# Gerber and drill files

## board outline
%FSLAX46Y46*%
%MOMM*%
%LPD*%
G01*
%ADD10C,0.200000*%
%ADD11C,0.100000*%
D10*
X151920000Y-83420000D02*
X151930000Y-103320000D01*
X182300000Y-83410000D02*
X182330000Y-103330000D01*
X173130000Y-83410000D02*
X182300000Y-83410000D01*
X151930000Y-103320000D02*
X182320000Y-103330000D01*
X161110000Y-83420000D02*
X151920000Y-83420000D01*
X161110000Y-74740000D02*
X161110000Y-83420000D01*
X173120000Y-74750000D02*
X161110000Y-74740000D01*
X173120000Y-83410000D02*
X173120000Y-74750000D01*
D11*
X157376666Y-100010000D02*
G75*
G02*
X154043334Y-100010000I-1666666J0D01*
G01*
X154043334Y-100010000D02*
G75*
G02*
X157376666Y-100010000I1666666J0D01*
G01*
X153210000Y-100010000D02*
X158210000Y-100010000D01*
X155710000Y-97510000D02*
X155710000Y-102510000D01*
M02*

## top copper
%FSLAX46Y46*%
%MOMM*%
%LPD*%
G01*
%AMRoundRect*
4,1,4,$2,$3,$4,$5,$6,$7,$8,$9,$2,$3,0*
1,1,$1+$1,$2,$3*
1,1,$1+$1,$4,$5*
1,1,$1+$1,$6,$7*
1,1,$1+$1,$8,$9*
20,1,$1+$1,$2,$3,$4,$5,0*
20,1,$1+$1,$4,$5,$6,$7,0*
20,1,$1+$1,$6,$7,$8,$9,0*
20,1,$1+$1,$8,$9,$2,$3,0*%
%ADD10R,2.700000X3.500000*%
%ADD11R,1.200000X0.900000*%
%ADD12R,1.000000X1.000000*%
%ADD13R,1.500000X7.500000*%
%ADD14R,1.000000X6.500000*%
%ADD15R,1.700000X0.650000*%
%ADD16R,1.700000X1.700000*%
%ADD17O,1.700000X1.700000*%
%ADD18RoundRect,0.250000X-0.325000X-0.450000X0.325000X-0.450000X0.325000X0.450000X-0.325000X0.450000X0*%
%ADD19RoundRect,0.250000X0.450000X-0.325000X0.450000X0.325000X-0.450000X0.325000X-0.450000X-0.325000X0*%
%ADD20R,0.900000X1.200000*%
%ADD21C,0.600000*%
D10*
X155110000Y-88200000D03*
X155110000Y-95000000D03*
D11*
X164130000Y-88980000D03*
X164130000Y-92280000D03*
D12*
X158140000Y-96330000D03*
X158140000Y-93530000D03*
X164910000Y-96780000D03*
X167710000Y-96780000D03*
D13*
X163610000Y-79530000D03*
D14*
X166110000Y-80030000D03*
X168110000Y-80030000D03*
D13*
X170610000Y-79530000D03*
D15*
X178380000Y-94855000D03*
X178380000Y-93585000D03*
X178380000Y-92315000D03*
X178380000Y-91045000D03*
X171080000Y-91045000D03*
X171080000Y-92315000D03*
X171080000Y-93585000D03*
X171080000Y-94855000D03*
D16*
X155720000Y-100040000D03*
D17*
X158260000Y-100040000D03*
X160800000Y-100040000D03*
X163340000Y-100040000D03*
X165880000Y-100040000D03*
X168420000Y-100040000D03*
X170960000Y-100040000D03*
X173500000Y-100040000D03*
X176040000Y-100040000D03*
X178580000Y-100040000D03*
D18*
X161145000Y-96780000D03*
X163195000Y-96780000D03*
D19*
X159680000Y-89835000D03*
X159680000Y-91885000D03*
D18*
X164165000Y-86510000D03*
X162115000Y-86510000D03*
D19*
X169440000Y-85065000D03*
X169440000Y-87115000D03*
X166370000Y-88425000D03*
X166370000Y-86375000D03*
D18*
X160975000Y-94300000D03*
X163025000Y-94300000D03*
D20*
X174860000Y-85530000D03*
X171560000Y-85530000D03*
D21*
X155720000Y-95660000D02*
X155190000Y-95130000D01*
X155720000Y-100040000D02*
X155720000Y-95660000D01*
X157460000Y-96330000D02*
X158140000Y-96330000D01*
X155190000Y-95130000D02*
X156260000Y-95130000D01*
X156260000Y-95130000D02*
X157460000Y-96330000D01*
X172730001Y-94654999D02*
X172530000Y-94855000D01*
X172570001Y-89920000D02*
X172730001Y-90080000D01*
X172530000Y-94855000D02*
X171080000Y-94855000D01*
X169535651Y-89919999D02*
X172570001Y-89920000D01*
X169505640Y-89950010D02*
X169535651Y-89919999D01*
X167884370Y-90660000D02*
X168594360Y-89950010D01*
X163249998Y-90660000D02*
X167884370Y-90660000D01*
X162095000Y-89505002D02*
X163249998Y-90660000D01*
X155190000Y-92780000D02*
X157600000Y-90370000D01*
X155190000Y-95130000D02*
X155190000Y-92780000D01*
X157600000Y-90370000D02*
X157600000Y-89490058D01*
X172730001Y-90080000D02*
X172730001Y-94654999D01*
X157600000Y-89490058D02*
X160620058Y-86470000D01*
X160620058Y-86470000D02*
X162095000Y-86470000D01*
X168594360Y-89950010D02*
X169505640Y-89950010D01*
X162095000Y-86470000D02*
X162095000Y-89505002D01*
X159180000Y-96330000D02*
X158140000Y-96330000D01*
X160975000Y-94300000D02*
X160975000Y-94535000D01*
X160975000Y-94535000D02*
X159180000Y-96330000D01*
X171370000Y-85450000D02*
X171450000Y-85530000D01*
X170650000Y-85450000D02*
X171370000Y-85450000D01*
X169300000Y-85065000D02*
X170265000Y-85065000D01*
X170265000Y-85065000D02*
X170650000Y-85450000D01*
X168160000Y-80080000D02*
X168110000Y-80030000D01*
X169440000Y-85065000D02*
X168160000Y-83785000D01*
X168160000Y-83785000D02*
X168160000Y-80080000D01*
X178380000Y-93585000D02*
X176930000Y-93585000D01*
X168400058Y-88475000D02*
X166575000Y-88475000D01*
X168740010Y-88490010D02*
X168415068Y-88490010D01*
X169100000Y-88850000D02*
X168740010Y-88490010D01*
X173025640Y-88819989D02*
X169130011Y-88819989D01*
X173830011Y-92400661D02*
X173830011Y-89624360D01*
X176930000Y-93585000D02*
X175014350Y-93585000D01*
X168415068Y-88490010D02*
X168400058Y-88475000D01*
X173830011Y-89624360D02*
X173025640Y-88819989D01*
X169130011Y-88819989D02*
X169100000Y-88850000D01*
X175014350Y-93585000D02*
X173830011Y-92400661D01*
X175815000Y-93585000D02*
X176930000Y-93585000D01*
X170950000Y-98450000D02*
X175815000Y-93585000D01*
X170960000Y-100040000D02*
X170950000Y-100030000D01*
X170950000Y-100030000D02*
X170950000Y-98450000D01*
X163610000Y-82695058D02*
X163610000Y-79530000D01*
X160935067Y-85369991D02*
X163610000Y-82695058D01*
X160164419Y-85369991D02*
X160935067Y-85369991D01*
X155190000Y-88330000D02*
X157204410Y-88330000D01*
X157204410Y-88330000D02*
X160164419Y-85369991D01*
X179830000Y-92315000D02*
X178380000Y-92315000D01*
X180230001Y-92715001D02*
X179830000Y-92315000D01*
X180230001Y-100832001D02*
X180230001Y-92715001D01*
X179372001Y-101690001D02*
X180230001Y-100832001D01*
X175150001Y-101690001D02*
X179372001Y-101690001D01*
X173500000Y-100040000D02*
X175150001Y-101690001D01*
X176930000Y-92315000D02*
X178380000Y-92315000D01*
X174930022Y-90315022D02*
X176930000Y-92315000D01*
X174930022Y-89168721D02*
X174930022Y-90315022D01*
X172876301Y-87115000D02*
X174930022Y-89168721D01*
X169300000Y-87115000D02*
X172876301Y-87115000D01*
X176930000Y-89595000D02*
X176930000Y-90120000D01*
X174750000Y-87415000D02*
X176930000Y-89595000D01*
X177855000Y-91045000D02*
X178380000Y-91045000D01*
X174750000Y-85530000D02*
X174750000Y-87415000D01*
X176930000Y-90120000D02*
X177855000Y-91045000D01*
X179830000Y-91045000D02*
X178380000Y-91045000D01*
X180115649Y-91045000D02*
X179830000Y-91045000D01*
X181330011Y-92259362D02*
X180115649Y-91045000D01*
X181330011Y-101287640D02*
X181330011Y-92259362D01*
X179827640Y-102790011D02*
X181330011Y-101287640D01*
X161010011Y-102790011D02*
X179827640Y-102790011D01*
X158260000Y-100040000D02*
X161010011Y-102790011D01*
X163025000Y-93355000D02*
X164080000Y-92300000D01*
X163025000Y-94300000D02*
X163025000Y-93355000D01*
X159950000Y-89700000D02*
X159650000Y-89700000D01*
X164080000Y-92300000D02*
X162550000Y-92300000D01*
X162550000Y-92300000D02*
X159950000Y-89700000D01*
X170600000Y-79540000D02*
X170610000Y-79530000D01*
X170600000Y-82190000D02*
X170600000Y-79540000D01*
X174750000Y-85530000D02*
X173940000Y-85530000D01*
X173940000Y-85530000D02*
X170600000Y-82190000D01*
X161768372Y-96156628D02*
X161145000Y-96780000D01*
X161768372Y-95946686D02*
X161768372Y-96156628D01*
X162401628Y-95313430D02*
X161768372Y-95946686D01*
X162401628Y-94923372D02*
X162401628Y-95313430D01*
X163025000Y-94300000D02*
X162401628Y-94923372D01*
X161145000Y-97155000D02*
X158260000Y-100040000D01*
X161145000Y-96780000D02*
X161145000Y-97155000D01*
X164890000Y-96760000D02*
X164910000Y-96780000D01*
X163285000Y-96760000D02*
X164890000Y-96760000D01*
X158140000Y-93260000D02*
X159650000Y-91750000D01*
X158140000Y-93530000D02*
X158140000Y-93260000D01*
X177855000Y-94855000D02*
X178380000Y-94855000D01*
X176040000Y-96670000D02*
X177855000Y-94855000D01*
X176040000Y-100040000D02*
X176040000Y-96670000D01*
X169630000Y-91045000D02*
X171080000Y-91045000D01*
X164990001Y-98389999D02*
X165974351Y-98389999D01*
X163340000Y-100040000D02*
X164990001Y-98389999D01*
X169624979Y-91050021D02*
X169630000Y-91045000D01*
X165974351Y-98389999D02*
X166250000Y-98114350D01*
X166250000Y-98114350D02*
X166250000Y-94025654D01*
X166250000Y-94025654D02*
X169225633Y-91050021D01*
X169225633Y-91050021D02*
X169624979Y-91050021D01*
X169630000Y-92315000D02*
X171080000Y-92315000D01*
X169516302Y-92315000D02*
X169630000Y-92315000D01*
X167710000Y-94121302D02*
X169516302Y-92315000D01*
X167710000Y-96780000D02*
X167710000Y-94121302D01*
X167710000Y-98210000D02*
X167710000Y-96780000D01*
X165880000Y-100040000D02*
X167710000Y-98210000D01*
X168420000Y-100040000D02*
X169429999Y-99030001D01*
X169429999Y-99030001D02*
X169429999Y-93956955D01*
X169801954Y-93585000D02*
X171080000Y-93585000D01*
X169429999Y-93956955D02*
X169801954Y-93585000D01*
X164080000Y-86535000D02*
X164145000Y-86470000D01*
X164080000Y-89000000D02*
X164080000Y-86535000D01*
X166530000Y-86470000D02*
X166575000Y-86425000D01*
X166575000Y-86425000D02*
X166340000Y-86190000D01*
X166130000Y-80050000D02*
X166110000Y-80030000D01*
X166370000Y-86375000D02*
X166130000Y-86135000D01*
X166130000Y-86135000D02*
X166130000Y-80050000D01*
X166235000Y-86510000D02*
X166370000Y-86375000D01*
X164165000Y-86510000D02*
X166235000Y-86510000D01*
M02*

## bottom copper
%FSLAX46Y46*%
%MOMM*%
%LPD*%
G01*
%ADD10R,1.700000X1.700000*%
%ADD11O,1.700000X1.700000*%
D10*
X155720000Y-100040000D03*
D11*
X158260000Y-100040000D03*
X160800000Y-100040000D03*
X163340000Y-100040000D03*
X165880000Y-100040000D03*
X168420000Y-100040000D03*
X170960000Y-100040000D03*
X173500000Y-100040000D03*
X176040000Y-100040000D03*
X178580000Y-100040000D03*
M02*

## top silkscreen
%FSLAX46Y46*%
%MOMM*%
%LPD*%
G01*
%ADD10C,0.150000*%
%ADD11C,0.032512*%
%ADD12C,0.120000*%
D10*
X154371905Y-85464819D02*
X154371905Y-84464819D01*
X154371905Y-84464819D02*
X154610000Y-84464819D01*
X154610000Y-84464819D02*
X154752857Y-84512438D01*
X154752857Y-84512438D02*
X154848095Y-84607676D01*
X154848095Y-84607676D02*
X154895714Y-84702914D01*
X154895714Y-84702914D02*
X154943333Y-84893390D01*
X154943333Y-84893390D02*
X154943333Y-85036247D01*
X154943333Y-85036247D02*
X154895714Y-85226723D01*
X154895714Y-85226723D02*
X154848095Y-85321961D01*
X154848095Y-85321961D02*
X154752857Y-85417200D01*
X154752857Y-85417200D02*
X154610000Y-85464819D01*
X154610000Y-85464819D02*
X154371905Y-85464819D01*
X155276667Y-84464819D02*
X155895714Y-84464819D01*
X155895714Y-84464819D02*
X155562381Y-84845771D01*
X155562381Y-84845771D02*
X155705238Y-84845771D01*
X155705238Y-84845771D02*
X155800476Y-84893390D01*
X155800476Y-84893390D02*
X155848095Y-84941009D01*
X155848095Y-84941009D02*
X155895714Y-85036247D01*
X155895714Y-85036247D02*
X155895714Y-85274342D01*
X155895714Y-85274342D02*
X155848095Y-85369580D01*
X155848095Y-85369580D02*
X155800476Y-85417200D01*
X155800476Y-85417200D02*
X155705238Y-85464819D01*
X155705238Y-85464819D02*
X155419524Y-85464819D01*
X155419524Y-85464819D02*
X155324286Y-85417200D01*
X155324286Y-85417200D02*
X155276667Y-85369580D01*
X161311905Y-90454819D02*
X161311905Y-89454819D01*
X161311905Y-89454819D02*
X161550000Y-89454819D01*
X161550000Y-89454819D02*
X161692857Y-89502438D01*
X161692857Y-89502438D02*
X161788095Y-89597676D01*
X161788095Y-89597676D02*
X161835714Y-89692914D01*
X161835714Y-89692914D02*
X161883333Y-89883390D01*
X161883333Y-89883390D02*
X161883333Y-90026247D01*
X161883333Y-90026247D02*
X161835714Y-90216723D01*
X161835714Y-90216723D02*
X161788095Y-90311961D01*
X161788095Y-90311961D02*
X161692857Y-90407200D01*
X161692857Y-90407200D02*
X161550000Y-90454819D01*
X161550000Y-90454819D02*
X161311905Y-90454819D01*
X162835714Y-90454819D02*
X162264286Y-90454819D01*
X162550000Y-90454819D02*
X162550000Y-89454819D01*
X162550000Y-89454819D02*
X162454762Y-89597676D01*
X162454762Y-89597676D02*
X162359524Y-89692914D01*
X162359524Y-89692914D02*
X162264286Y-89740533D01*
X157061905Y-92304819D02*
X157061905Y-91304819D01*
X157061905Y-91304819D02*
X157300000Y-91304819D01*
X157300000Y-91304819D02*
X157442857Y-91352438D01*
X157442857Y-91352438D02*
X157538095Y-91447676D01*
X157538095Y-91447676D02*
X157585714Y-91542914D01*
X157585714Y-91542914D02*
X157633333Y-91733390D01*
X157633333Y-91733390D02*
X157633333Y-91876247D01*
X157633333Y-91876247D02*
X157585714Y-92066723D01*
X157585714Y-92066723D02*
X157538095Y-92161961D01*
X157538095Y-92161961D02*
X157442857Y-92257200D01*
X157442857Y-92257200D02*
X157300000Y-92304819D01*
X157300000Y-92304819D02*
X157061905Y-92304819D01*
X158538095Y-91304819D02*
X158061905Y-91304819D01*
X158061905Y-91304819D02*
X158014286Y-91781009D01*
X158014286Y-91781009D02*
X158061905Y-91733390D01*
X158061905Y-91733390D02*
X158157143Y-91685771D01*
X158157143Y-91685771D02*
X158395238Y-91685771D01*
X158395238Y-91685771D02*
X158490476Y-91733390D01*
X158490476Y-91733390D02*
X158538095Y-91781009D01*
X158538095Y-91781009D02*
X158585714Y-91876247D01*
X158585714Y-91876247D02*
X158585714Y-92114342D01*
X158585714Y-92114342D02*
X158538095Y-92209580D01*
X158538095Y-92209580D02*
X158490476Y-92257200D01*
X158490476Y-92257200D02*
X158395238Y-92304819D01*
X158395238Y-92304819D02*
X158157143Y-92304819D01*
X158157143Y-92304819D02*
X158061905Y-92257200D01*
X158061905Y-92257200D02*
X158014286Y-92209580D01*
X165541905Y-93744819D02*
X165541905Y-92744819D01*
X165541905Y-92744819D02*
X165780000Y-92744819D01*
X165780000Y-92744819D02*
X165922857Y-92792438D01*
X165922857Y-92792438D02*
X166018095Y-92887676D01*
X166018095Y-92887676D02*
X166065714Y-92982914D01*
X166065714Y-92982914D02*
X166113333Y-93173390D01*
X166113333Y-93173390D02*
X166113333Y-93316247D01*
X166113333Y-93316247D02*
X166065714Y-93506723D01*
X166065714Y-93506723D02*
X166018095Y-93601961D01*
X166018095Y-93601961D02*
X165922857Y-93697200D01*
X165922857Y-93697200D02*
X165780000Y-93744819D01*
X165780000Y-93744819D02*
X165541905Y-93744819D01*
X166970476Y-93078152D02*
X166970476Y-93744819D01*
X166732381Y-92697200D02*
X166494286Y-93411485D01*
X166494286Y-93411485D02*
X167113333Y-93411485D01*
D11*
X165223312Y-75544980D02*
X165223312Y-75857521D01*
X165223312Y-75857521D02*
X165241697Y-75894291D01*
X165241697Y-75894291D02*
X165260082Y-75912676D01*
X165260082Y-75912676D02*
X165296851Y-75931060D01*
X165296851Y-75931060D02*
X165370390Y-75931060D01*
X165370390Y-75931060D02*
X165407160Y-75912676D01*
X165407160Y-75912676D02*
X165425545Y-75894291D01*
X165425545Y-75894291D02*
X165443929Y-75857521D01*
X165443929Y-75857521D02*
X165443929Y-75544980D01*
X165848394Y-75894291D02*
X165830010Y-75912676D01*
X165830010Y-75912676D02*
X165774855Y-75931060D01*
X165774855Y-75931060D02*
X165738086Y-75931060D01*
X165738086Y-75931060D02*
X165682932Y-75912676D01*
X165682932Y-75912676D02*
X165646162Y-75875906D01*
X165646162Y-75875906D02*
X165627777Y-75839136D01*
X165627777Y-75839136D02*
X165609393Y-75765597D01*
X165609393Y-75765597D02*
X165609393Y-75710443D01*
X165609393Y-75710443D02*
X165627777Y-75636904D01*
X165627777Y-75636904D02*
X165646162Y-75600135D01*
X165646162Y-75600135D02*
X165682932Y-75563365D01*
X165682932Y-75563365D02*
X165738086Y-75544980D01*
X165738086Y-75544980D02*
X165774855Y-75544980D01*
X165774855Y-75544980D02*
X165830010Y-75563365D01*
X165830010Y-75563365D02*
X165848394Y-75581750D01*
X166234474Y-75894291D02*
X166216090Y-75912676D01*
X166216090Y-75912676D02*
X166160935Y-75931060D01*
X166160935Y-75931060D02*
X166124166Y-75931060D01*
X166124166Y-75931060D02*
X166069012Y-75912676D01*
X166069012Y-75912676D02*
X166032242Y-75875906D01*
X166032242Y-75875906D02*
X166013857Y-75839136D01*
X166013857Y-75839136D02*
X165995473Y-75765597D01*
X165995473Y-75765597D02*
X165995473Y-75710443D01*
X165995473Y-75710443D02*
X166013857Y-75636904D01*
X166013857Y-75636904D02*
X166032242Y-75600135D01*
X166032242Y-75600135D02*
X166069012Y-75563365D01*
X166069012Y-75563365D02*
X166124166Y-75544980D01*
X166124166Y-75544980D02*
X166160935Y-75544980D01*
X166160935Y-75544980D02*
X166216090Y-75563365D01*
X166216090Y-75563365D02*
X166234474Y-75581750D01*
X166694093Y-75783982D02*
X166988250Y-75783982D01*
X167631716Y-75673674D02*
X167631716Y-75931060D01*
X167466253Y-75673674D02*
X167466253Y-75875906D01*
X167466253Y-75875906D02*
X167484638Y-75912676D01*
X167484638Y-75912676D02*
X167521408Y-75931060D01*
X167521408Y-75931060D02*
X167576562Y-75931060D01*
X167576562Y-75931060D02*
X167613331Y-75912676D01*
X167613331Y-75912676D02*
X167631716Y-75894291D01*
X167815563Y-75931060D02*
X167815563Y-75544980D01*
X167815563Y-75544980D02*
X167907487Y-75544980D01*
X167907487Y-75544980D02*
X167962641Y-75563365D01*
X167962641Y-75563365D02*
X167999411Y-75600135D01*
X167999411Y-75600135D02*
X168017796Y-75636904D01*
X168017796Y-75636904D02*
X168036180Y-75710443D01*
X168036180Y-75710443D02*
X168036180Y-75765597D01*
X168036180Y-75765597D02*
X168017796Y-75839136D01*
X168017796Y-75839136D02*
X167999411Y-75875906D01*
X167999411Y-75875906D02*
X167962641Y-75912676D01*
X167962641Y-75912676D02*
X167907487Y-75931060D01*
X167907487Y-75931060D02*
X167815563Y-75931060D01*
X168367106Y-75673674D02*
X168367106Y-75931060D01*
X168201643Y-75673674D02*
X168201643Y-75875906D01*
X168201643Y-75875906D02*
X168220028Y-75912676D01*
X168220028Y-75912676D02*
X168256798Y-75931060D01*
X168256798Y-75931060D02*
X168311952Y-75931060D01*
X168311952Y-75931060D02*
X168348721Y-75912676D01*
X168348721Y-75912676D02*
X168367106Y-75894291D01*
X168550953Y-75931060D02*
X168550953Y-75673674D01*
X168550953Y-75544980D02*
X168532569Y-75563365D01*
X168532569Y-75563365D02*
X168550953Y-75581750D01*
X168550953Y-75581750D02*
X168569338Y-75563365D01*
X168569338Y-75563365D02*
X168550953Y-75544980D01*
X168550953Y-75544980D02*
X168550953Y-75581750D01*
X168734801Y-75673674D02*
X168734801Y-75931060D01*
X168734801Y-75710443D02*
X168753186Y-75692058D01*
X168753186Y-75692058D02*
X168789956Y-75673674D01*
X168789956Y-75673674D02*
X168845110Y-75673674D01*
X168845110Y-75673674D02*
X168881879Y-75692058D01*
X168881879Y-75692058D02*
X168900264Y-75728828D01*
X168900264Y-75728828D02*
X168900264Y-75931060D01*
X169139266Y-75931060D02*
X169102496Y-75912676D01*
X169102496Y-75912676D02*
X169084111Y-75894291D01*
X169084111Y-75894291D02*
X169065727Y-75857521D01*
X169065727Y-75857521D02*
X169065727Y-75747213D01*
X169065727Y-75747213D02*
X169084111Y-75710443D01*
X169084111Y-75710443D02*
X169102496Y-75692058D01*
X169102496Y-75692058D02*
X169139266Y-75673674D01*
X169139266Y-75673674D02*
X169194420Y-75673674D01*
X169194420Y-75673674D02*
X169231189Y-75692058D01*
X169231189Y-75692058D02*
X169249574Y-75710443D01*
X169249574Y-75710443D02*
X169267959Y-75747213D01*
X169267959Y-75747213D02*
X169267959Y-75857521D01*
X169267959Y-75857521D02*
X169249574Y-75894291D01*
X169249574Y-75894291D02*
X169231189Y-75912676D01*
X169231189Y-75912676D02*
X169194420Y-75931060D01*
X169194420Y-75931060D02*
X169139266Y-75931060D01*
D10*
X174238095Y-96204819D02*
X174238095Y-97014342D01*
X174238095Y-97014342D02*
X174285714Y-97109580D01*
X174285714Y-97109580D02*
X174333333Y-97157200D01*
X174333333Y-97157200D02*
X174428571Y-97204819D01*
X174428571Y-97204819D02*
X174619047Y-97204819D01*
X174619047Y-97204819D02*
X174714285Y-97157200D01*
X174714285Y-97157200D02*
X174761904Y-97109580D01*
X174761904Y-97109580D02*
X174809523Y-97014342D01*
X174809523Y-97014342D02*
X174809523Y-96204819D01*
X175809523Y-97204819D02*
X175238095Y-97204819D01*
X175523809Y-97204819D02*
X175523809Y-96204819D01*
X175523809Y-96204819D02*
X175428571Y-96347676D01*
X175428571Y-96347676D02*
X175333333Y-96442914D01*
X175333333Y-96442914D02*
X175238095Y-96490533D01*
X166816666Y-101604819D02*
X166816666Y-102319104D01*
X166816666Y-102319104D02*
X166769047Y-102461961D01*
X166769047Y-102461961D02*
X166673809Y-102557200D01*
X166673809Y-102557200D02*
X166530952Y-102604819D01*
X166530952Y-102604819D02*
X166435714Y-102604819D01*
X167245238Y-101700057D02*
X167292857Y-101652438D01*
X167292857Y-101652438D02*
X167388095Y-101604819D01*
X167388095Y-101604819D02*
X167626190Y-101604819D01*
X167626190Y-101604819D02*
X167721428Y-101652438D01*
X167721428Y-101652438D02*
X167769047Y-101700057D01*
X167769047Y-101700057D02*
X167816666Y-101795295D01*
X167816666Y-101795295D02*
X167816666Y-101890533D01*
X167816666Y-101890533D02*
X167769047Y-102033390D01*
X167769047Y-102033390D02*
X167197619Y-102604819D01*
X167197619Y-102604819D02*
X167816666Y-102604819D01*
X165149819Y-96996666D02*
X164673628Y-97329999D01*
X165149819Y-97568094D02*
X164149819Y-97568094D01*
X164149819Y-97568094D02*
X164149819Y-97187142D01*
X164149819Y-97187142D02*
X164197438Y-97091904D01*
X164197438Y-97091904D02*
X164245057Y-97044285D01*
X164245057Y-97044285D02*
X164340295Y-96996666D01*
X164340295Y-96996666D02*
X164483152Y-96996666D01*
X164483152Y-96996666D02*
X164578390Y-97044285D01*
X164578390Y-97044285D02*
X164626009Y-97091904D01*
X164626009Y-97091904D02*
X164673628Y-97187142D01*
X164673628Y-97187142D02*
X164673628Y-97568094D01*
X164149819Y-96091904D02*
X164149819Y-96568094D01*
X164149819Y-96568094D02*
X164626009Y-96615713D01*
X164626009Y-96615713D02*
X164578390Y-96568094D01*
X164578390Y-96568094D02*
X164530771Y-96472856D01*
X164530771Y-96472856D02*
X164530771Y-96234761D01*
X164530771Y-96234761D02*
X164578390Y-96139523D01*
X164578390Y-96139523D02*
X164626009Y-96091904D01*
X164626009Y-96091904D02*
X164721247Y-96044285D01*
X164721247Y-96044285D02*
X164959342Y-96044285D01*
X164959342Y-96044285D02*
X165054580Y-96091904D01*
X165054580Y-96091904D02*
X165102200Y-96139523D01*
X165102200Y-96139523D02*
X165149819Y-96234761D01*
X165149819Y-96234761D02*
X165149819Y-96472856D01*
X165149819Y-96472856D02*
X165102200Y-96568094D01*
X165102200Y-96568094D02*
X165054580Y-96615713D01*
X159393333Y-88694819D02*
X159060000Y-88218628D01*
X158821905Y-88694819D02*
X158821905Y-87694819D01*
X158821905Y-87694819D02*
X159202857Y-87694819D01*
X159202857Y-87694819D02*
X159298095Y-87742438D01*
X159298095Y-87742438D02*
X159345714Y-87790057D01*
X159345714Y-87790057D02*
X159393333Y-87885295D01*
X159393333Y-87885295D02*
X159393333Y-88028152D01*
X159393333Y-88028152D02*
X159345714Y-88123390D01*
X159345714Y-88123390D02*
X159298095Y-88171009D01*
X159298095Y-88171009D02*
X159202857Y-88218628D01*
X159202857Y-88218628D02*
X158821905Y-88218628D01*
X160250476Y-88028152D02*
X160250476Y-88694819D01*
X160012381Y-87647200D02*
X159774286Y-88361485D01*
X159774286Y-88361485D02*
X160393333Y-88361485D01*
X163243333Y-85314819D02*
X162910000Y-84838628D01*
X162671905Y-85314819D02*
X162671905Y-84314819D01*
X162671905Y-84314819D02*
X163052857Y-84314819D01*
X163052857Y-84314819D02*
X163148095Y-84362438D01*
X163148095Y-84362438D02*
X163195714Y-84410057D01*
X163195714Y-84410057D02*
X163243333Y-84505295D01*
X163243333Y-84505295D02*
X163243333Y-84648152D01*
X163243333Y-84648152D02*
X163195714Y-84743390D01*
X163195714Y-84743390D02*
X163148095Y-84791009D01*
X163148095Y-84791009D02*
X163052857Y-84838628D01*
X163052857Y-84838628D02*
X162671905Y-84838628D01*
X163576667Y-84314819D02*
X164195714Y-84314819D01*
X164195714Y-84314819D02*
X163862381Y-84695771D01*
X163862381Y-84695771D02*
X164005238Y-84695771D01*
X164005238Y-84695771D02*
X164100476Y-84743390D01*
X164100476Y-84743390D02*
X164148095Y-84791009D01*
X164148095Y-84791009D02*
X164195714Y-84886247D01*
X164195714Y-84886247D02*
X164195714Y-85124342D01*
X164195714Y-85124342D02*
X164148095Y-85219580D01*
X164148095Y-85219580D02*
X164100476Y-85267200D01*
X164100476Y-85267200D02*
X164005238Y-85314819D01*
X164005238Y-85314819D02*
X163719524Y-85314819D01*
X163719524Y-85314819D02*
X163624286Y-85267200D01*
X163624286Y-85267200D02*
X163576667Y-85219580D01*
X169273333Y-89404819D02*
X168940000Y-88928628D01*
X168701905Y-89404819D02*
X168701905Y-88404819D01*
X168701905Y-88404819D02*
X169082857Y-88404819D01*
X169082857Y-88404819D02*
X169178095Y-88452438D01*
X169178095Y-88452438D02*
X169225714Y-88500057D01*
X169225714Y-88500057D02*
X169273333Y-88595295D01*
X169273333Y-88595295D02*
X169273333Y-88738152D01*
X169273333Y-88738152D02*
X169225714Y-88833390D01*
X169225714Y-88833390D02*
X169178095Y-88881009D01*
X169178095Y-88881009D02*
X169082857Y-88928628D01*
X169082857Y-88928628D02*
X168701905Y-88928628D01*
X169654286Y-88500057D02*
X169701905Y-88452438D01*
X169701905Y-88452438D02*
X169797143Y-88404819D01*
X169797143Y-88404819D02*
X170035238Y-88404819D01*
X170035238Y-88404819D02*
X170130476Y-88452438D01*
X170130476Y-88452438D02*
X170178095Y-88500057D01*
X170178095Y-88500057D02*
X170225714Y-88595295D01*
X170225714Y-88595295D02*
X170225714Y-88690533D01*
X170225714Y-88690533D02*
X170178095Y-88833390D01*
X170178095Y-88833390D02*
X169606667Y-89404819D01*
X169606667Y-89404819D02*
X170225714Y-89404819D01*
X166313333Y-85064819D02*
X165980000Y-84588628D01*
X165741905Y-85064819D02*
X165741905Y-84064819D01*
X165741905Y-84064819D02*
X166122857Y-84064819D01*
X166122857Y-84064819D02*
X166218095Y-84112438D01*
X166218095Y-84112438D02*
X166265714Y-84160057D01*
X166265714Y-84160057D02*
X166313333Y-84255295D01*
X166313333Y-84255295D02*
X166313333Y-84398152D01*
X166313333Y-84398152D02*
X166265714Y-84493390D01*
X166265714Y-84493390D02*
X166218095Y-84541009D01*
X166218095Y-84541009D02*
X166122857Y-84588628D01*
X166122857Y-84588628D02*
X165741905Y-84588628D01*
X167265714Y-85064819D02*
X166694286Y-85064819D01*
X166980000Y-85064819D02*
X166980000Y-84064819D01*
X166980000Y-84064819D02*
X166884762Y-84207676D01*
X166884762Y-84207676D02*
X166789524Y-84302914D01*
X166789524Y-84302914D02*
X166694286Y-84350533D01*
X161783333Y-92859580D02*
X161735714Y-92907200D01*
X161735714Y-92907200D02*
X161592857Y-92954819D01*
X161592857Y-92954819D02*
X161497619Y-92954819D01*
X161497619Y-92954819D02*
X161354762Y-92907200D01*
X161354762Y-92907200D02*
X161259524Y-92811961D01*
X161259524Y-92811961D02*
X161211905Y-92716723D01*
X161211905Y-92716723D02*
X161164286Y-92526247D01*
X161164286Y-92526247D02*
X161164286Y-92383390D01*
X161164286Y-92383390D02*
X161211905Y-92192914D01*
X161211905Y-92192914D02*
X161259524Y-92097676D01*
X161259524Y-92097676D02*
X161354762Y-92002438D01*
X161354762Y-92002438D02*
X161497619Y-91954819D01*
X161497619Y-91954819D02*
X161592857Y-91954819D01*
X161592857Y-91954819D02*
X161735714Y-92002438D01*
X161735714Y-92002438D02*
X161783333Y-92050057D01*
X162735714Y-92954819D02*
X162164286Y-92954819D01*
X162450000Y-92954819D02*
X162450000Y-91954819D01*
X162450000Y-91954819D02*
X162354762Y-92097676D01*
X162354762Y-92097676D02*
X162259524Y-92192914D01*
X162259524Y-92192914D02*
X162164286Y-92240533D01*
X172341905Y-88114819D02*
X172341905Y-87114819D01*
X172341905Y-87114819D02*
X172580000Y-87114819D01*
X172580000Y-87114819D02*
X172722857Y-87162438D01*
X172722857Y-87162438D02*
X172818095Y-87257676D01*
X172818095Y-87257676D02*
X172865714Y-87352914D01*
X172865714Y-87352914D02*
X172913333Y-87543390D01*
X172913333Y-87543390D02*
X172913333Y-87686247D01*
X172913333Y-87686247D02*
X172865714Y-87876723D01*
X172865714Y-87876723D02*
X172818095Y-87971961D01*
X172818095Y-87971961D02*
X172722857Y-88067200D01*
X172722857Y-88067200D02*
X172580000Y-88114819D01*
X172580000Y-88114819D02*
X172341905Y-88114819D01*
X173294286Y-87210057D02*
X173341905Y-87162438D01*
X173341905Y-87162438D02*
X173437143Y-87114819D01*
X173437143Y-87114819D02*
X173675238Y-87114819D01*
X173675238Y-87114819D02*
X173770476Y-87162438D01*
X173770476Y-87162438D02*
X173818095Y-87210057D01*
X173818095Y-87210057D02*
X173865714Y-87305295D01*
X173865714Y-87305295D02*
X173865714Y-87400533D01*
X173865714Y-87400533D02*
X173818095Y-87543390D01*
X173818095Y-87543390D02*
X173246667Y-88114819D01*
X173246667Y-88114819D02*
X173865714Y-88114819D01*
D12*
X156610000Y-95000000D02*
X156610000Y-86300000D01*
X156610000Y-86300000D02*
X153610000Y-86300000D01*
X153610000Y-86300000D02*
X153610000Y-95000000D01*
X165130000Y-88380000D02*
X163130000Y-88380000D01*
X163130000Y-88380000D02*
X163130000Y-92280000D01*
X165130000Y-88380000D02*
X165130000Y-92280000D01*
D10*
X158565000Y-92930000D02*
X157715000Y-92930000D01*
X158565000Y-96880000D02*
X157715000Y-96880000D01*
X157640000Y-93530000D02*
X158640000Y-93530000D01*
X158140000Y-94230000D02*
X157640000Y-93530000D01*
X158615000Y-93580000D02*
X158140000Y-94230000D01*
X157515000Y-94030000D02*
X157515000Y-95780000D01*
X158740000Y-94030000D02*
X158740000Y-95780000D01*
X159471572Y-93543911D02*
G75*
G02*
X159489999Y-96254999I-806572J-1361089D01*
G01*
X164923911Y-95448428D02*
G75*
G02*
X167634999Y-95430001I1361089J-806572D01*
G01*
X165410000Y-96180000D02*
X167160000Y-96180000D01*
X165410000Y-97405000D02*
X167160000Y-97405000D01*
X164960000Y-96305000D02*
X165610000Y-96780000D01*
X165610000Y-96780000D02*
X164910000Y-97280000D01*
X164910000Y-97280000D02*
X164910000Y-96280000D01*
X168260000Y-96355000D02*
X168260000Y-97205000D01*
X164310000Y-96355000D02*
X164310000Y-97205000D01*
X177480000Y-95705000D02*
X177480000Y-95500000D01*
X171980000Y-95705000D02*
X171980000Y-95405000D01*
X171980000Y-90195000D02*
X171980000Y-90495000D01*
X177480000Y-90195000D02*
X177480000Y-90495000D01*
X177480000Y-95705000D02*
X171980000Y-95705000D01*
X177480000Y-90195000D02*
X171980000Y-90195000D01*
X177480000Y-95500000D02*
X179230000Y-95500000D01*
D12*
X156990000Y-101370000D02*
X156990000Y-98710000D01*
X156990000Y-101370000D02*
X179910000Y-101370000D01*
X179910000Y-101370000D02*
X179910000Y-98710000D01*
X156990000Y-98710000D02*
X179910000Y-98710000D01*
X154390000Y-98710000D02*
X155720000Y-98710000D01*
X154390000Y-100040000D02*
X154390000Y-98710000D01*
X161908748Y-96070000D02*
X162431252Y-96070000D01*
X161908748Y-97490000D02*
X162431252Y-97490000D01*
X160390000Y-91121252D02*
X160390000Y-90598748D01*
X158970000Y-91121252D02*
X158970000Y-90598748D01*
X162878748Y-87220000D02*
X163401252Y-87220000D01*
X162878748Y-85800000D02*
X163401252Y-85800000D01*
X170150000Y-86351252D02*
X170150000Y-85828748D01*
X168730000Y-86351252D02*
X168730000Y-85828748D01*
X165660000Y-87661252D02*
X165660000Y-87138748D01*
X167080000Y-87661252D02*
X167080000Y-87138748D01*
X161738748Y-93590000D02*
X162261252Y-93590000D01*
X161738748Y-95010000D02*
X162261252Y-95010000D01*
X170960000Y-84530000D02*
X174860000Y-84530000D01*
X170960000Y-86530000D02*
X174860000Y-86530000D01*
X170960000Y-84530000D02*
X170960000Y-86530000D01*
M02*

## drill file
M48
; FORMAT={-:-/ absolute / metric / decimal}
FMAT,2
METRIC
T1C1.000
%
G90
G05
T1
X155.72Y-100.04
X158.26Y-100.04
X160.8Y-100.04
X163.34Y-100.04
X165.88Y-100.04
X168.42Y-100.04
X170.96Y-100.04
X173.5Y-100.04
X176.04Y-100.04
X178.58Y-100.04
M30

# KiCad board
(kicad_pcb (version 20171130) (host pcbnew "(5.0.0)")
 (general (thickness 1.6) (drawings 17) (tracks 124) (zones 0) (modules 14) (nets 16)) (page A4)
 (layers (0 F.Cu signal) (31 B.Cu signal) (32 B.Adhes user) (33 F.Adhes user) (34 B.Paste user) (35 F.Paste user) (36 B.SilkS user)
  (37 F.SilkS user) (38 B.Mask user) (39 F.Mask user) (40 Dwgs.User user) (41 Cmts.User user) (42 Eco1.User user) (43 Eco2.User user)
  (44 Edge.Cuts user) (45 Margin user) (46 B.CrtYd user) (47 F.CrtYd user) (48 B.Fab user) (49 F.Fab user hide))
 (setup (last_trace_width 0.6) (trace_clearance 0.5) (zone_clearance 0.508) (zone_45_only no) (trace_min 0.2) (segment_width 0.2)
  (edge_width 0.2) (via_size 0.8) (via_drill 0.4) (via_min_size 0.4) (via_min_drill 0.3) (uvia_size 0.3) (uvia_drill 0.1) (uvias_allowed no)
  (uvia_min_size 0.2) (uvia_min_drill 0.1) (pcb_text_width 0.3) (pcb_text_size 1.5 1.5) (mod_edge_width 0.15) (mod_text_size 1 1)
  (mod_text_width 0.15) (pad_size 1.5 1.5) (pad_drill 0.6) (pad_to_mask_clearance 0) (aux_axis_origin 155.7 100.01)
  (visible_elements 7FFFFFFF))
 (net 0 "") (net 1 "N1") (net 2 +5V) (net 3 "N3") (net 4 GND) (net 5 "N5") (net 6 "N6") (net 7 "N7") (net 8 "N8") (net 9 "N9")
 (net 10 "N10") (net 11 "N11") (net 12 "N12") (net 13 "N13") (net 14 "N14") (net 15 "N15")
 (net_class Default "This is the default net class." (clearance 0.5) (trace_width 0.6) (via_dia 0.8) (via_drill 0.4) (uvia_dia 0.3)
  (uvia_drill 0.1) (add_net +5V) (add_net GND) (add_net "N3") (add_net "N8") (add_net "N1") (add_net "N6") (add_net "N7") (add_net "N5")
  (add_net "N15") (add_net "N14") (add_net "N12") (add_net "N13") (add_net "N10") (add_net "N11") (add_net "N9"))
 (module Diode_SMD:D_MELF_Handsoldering (layer F.Cu) (at 155.11 91.6 270)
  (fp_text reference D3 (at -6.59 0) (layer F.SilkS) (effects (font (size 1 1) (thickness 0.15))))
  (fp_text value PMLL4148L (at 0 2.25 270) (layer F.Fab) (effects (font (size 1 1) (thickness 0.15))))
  (fp_line (start 3.4 -1.5) (end -5.3 -1.5) (layer F.SilkS) (width 0.12))
  (fp_line (start -5.3 -1.5) (end -5.3 1.5) (layer F.SilkS) (width 0.12))
  (fp_line (start -5.3 1.5) (end 3.4 1.5) (layer F.SilkS) (width 0.12))
  (pad 1 smd rect (at -3.4 0 270) (size 3.5 2.7) (layers F.Cu F.Paste F.Mask) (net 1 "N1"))
  (pad 2 smd rect (at 3.4 0 270) (size 3.5 2.7) (layers F.Cu F.Paste F.Mask) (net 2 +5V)))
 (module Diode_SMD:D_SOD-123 (layer F.Cu) (at 164.13 90.63 270)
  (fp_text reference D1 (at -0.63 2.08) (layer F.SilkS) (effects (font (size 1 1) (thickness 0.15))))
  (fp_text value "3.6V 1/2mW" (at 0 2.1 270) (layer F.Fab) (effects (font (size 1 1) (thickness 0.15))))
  (fp_line (start -2.25 -1) (end -2.25 1) (layer F.SilkS) (width 0.12))
  (fp_line (start -2.25 1) (end 1.65 1) (layer F.SilkS) (width 0.12))
  (fp_line (start -2.25 -1) (end 1.65 -1) (layer F.SilkS) (width 0.12))
  (pad 1 smd rect (at -1.65 0 270) (size 0.9 1.2) (layers F.Cu F.Paste F.Mask) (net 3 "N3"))
  (pad 2 smd rect (at 1.65 0 270) (size 0.9 1.2) (layers F.Cu F.Paste F.Mask) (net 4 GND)))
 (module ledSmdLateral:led (layer F.Cu) (at 158.14 95.33 270)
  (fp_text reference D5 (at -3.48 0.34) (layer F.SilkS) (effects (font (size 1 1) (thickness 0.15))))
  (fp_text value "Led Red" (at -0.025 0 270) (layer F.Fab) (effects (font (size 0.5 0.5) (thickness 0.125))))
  (fp_line (start -2.4 -0.425) (end -2.4 0.425) (layer F.SilkS) (width 0.15))
  (fp_line (start 1.55 -0.425) (end 1.55 0.425) (layer F.SilkS) (width 0.15))
  (fp_line (start -1.8 0.5) (end -1.8 -0.5) (layer F.SilkS) (width 0.15))
  (fp_line (start -1.1 0) (end -1.8 0.5) (layer F.SilkS) (width 0.15))
  (fp_line (start -1.75 -0.475) (end -1.1 0) (layer F.SilkS) (width 0.15))
  (fp_line (start -1.3 0.625) (end 0.45 0.625) (layer F.SilkS) (width 0.15))
  (fp_line (start -1.3 -0.6) (end 0.45 -0.6) (layer F.SilkS) (width 0.15))
  (fp_arc (start -0.425 -0.525) (end 0.924999 -1.349999) (angle -117.9197664) (layer F.SilkS) (width 0.15))
  (pad 2 smd rect (at 1 0 270) (size 1 1) (layers F.Cu F.Paste F.Mask) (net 2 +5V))
  (pad 1 smd rect (at -1.8 0 270) (size 1 1) (layers F.Cu F.Paste F.Mask) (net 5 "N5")))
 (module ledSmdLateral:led (layer F.Cu) (at 166.71 96.78)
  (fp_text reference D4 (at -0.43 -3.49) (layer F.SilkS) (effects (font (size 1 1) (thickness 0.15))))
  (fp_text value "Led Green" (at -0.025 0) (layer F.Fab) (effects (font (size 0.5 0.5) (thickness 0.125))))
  (fp_arc (start -0.425 -0.525) (end 0.924999 -1.349999) (angle -117.9197664) (layer F.SilkS) (width 0.15))
  (fp_line (start -1.3 -0.6) (end 0.45 -0.6) (layer F.SilkS) (width 0.15))
  (fp_line (start -1.3 0.625) (end 0.45 0.625) (layer F.SilkS) (width 0.15))
  (fp_line (start -1.75 -0.475) (end -1.1 0) (layer F.SilkS) (width 0.15))
  (fp_line (start -1.1 0) (end -1.8 0.5) (layer F.SilkS) (width 0.15))
  (fp_line (start -1.8 0.5) (end -1.8 -0.5) (layer F.SilkS) (width 0.15))
  (fp_line (start 1.55 -0.425) (end 1.55 0.425) (layer F.SilkS) (width 0.15))
  (fp_line (start -2.4 -0.425) (end -2.4 0.425) (layer F.SilkS) (width 0.15))
  (pad 1 smd rect (at -1.8 0) (size 1 1) (layers F.Cu F.Paste F.Mask) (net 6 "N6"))
  (pad 2 smd rect (at 1 0) (size 1 1) (layers F.Cu F.Paste F.Mask) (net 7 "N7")))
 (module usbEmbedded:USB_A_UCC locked (layer F.Cu) (at 167.11 79.73 270)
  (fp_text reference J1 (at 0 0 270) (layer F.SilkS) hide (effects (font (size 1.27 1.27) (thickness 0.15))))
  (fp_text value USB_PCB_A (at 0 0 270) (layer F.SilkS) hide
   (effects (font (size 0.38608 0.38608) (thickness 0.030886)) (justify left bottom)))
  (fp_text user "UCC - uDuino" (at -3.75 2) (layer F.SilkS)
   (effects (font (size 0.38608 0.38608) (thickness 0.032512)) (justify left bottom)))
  (pad 1 smd rect (at -0.2 3.5 270) (size 7.5 1.5) (layers F.Cu F.Paste F.Mask) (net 1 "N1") (solder_mask_margin 0.1016))
  (pad 2 smd rect (at 0.3 1 270) (size 6.5 1) (layers F.Cu F.Paste F.Mask) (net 3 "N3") (solder_mask_margin 0.1016))
  (pad 3 smd rect (at 0.3 -1 270) (size 6.5 1) (layers F.Cu F.Paste F.Mask) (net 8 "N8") (solder_mask_margin 0.1016))
  (pad 4 smd rect (at -0.2 -3.5 270) (size 7.5 1.5) (layers F.Cu F.Paste F.Mask) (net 4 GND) (solder_mask_margin 0.1016)))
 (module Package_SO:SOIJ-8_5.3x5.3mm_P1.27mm (layer F.Cu) (at 174.73 92.95 180)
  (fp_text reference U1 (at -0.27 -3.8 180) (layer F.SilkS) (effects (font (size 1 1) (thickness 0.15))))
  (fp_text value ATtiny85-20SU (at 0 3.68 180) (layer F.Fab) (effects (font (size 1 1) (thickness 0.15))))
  (fp_line (start -2.75 -2.755) (end -2.75 -2.55) (layer F.SilkS) (width 0.15))
  (fp_line (start 2.75 -2.755) (end 2.75 -2.455) (layer F.SilkS) (width 0.15))
  (fp_line (start 2.75 2.755) (end 2.75 2.455) (layer F.SilkS) (width 0.15))
  (fp_line (start -2.75 2.755) (end -2.75 2.455) (layer F.SilkS) (width 0.15))
  (fp_line (start -2.75 -2.755) (end 2.75 -2.755) (layer F.SilkS) (width 0.15))
  (fp_line (start -2.75 2.755) (end 2.75 2.755) (layer F.SilkS) (width 0.15))
  (fp_line (start -2.75 -2.55) (end -4.5 -2.55) (layer F.SilkS) (width 0.15))
  (pad 1 smd rect (at -3.65 -1.905 180) (size 1.7 0.65) (layers F.Cu F.Paste F.Mask) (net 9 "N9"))
  (pad 2 smd rect (at -3.65 -0.635 180) (size 1.7 0.65) (layers F.Cu F.Paste F.Mask) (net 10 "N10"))
  (pad 3 smd rect (at -3.65 0.635 180) (size 1.7 0.65) (layers F.Cu F.Paste F.Mask) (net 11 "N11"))
  (pad 4 smd rect (at -3.65 1.905 180) (size 1.7 0.65) (layers F.Cu F.Paste F.Mask) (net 4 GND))
  (pad 5 smd rect (at 3.65 1.905 180) (size 1.7 0.65) (layers F.Cu F.Paste F.Mask) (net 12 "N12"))
  (pad 6 smd rect (at 3.65 0.635 180) (size 1.7 0.65) (layers F.Cu F.Paste F.Mask) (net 7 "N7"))
  (pad 7 smd rect (at 3.65 -0.635 180) (size 1.7 0.65) (layers F.Cu F.Paste F.Mask) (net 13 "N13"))
  (pad 8 smd rect (at 3.65 -1.905 180) (size 1.7 0.65) (layers F.Cu F.Paste F.Mask) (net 2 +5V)))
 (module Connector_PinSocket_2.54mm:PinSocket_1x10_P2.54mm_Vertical (layer F.Cu) (at 155.72 100.04 90)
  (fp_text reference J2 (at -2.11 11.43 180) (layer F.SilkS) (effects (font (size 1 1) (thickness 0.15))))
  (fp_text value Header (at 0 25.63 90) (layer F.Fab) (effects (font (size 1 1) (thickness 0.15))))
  (fp_line (start -1.33 1.27) (end 1.33 1.27) (layer F.SilkS) (width 0.12))
  (fp_line (start -1.33 1.27) (end -1.33 24.19) (layer F.SilkS) (width 0.12))
  (fp_line (start -1.33 24.19) (end 1.33 24.19) (layer F.SilkS) (width 0.12))
  (fp_line (start 1.33 1.27) (end 1.33 24.19) (layer F.SilkS) (width 0.12))
  (fp_line (start 1.33 -1.33) (end 1.33 0) (layer F.SilkS) (width 0.12))
  (fp_line (start 0 -1.33) (end 1.33 -1.33) (layer F.SilkS) (width 0.12))
  (pad 1 thru_hole rect (at 0 0 90) (size 1.7 1.7) (drill 1) (layers *.Cu *.Mask) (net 2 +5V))
  (pad 2 thru_hole oval (at 0 2.54 90) (size 1.7 1.7) (drill 1) (layers *.Cu *.Mask) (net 4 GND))
  (pad 3 thru_hole oval (at 0 5.08 90) (size 1.7 1.7) (drill 1) (layers *.Cu *.Mask) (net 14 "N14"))
  (pad 4 thru_hole oval (at 0 7.62 90) (size 1.7 1.7) (drill 1) (layers *.Cu *.Mask) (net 12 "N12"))
  (pad 5 thru_hole oval (at 0 10.16 90) (size 1.7 1.7) (drill 1) (layers *.Cu *.Mask) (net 7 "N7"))
  (pad 6 thru_hole oval (at 0 12.7 90) (size 1.7 1.7) (drill 1) (layers *.Cu *.Mask) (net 13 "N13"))
  (pad 7 thru_hole oval (at 0 15.24 90) (size 1.7 1.7) (drill 1) (layers *.Cu *.Mask) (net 10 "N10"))
  (pad 8 thru_hole oval (at 0 17.78 90) (size 1.7 1.7) (drill 1) (layers *.Cu *.Mask) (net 11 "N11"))
  (pad 9 thru_hole oval (at 0 20.32 90) (size 1.7 1.7) (drill 1) (layers *.Cu *.Mask) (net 9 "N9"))
  (pad 10 thru_hole oval (at 0 22.86 90) (size 1.7 1.7) (drill 1) (layers *.Cu *.Mask) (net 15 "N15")))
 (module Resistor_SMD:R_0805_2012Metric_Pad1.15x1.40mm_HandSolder (layer F.Cu) (at 162.17 96.78)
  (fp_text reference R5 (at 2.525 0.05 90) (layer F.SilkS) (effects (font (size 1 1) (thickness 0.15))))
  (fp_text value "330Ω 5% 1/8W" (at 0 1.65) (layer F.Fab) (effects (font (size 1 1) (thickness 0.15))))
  (fp_line (start -0.261252 -0.71) (end 0.261252 -0.71) (layer F.SilkS) (width 0.12))
  (fp_line (start -0.261252 0.71) (end 0.261252 0.71) (layer F.SilkS) (width 0.12))
  (pad 1 smd roundrect (at -1.025 0) (size 1.15 1.4) (layers F.Cu F.Paste F.Mask) (roundrect_rratio 0.217391) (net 4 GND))
  (pad 2 smd roundrect (at 1.025 0) (size 1.15 1.4) (layers F.Cu F.Paste F.Mask) (roundrect_rratio 0.217391) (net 6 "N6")))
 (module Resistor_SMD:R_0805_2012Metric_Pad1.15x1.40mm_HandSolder (layer F.Cu) (at 159.68 90.86 90)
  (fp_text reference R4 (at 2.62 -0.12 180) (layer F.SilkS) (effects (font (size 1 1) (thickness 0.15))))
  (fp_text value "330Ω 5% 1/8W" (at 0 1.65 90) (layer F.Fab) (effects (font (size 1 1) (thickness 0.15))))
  (fp_line (start -0.261252 0.71) (end 0.261252 0.71) (layer F.SilkS) (width 0.12))
  (fp_line (start -0.261252 -0.71) (end 0.261252 -0.71) (layer F.SilkS) (width 0.12))
  (pad 2 smd roundrect (at 1.025 0 90) (size 1.15 1.4) (layers F.Cu F.Paste F.Mask) (roundrect_rratio 0.217391) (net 4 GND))
  (pad 1 smd roundrect (at -1.025 0 90) (size 1.15 1.4) (layers F.Cu F.Paste F.Mask) (roundrect_rratio 0.217391) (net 5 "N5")))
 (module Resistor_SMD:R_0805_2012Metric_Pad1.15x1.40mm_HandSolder (layer F.Cu) (at 163.14 86.51)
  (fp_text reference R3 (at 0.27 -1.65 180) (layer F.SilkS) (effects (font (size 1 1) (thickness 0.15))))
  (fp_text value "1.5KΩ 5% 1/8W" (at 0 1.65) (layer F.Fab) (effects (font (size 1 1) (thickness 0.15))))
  (fp_line (start -0.261252 0.71) (end 0.261252 0.71) (layer F.SilkS) (width 0.12))
  (fp_line (start -0.261252 -0.71) (end 0.261252 -0.71) (layer F.SilkS) (width 0.12))
  (pad 2 smd roundrect (at 1.025 0) (size 1.15 1.4) (layers F.Cu F.Paste F.Mask) (roundrect_rratio 0.217391) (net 3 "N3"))
  (pad 1 smd roundrect (at -1.025 0) (size 1.15 1.4) (layers F.Cu F.Paste F.Mask) (roundrect_rratio 0.217391) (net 2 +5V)))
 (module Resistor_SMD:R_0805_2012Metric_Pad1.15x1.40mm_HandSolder (layer F.Cu) (at 169.44 86.09 90)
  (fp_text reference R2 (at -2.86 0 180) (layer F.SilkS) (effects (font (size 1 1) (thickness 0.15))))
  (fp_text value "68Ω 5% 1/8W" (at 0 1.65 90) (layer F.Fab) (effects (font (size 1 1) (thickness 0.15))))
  (fp_line (start -0.261252 0.71) (end 0.261252 0.71) (layer F.SilkS) (width 0.12))
  (fp_line (start -0.261252 -0.71) (end 0.261252 -0.71) (layer F.SilkS) (width 0.12))
  (pad 2 smd roundrect (at 1.025 0 90) (size 1.15 1.4) (layers F.Cu F.Paste F.Mask) (roundrect_rratio 0.217391) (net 8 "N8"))
  (pad 1 smd roundrect (at -1.025 0 90) (size 1.15 1.4) (layers F.Cu F.Paste F.Mask) (roundrect_rratio 0.217391) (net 11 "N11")))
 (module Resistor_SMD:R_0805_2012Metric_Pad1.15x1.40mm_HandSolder (layer F.Cu) (at 166.37 87.4 90)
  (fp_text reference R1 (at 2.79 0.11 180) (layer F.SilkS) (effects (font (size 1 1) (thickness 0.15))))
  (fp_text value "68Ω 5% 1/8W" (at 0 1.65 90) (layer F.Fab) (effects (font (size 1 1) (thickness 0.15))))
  (fp_line (start -0.261252 -0.71) (end 0.261252 -0.71) (layer F.SilkS) (width 0.12))
  (fp_line (start -0.261252 0.71) (end 0.261252 0.71) (layer F.SilkS) (width 0.12))
  (pad 1 smd roundrect (at -1.025 0 90) (size 1.15 1.4) (layers F.Cu F.Paste F.Mask) (roundrect_rratio 0.217391) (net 10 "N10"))
  (pad 2 smd roundrect (at 1.025 0 90) (size 1.15 1.4) (layers F.Cu F.Paste F.Mask) (roundrect_rratio 0.217391) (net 3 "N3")))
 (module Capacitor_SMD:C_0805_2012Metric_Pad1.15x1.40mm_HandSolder (layer F.Cu) (at 162 94.3)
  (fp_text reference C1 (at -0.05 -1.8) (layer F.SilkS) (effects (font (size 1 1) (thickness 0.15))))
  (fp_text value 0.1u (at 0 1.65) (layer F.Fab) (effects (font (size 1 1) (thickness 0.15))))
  (fp_line (start -0.261252 -0.71) (end 0.261252 -0.71) (layer F.SilkS) (width 0.12))
  (fp_line (start -0.261252 0.71) (end 0.261252 0.71) (layer F.SilkS) (width 0.12))
  (pad 1 smd roundrect (at -1.025 0) (size 1.15 1.4) (layers F.Cu F.Paste F.Mask) (roundrect_rratio 0.217391) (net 2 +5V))
  (pad 2 smd roundrect (at 1.025 0) (size 1.15 1.4) (layers F.Cu F.Paste F.Mask) (roundrect_rratio 0.217391) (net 4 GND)))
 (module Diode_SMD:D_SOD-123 (layer F.Cu) (at 173.21 85.53)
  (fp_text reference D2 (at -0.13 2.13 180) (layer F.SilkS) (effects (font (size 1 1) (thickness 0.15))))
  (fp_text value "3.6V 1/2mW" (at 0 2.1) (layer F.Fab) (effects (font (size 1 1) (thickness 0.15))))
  (fp_line (start -2.25 -1) (end 1.65 -1) (layer F.SilkS) (width 0.12))
  (fp_line (start -2.25 1) (end 1.65 1) (layer F.SilkS) (width 0.12))
  (fp_line (start -2.25 -1) (end -2.25 1) (layer F.SilkS) (width 0.12))
  (pad 2 smd rect (at 1.65 0) (size 0.9 1.2) (layers F.Cu F.Paste F.Mask) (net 4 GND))
  (pad 1 smd rect (at -1.65 0) (size 0.9 1.2) (layers F.Cu F.Paste F.Mask) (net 8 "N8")))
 (gr_line (start 151.92 83.42) (end 151.93 103.32) (layer Edge.Cuts) (width 0.2))
 (gr_line (start 182.3 83.41) (end 182.33 103.33) (layer Edge.Cuts) (width 0.2))
 (gr_line (start 173.13 83.41) (end 182.3 83.41) (layer Edge.Cuts) (width 0.2))
 (gr_line (start 151.93 103.32) (end 182.32 103.33) (layer Edge.Cuts) (width 0.2))
 (gr_line (start 161.11 83.42) (end 151.92 83.42) (layer Edge.Cuts) (width 0.2))
 (gr_line (start 161.11 74.74) (end 161.11 83.42) (layer Edge.Cuts) (width 0.2))
 (gr_line (start 173.12 74.75) (end 161.11 74.74) (layer Edge.Cuts) (width 0.2))
 (gr_line (start 173.12 83.41) (end 173.12 74.75) (layer Edge.Cuts) (width 0.2))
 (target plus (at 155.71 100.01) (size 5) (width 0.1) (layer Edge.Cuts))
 (segment (start 155.72 95.66) (end 155.19 95.13) (width 0.6) (layer F.Cu) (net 2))
 (segment (start 155.72 100.04) (end 155.72 95.66) (width 0.6) (layer F.Cu) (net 2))
 (segment (start 157.46 96.33) (end 158.14 96.33) (width 0.6) (layer F.Cu) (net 2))
 (segment (start 155.19 95.13) (end 156.26 95.13) (width 0.6) (layer F.Cu) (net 2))
 (segment (start 156.26 95.13) (end 157.46 96.33) (width 0.6) (layer F.Cu) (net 2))
 (segment (start 172.730001 94.654999) (end 172.53 94.855) (width 0.6) (layer F.Cu) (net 2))
 (segment (start 172.570001 89.92) (end 172.730001 90.08) (width 0.6) (layer F.Cu) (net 2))
 (segment (start 172.53 94.855) (end 171.08 94.855) (width 0.6) (layer F.Cu) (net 2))
 (segment (start 169.535651 89.919999) (end 172.570001 89.92) (width 0.6) (layer F.Cu) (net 2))
 (segment (start 169.50564 89.95001) (end 169.535651 89.919999) (width 0.6) (layer F.Cu) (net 2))
 (segment (start 167.88437 90.66) (end 168.59436 89.95001) (width 0.6) (layer F.Cu) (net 2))
 (segment (start 163.249998 90.66) (end 167.88437 90.66) (width 0.6) (layer F.Cu) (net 2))
 (segment (start 162.095 89.505002) (end 163.249998 90.66) (width 0.6) (layer F.Cu) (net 2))
 (segment (start 155.19 92.78) (end 157.6 90.37) (width 0.6) (layer F.Cu) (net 2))
 (segment (start 155.19 95.13) (end 155.19 92.78) (width 0.6) (layer F.Cu) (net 2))
 (segment (start 157.6 90.37) (end 157.6 89.490058) (width 0.6) (layer F.Cu) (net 2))
 (segment (start 172.730001 90.08) (end 172.730001 94.654999) (width 0.6) (layer F.Cu) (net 2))
 (segment (start 157.6 89.490058) (end 160.620058 86.47) (width 0.6) (layer F.Cu) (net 2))
 (segment (start 160.620058 86.47) (end 162.095 86.47) (width 0.6) (layer F.Cu) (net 2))
 (segment (start 168.59436 89.95001) (end 169.50564 89.95001) (width 0.6) (layer F.Cu) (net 2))
 (segment (start 162.095 86.47) (end 162.095 89.505002) (width 0.6) (layer F.Cu) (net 2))
 (segment (start 159.18 96.33) (end 158.14 96.33) (width 0.6) (layer F.Cu) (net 2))
 (segment (start 160.975 94.3) (end 160.975 94.535) (width 0.6) (layer F.Cu) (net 2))
 (segment (start 160.975 94.535) (end 159.18 96.33) (width 0.6) (layer F.Cu) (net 2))
 (segment (start 171.37 85.45) (end 171.45 85.53) (width 0.6) (layer F.Cu) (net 8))
 (segment (start 170.65 85.45) (end 171.37 85.45) (width 0.6) (layer F.Cu) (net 8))
 (segment (start 169.3 85.065) (end 170.265 85.065) (width 0.6) (layer F.Cu) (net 8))
 (segment (start 170.265 85.065) (end 170.65 85.45) (width 0.6) (layer F.Cu) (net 8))
 (segment (start 168.16 80.08) (end 168.11 80.03) (width 0.6) (layer F.Cu) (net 8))
 (segment (start 169.44 85.065) (end 168.16 83.785) (width 0.6) (layer F.Cu) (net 8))
 (segment (start 168.16 83.785) (end 168.16 80.08) (width 0.6) (layer F.Cu) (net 8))
 (segment (start 178.38 93.585) (end 176.93 93.585) (width 0.6) (layer F.Cu) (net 10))
 (segment (start 168.400058 88.475) (end 166.575 88.475) (width 0.6) (layer F.Cu) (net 10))
 (segment (start 168.74001 88.49001) (end 168.415068 88.49001) (width 0.6) (layer F.Cu) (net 10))
 (segment (start 169.1 88.85) (end 168.74001 88.49001) (width 0.6) (layer F.Cu) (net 10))
 (segment (start 173.02564 88.819989) (end 169.130011 88.819989) (width 0.6) (layer F.Cu) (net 10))
 (segment (start 173.830011 92.400661) (end 173.830011 89.62436) (width 0.6) (layer F.Cu) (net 10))
 (segment (start 176.93 93.585) (end 175.01435 93.585) (width 0.6) (layer F.Cu) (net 10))
 (segment (start 168.415068 88.49001) (end 168.400058 88.475) (width 0.6) (layer F.Cu) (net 10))
 (segment (start 173.830011 89.62436) (end 173.02564 88.819989) (width 0.6) (layer F.Cu) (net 10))
 (segment (start 169.130011 88.819989) (end 169.1 88.85) (width 0.6) (layer F.Cu) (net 10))
 (segment (start 175.01435 93.585) (end 173.830011 92.400661) (width 0.6) (layer F.Cu) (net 10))
 (segment (start 175.815 93.585) (end 176.93 93.585) (width 0.6) (layer F.Cu) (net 10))
 (segment (start 170.95 98.45) (end 175.815 93.585) (width 0.6) (layer F.Cu) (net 10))
 (segment (start 170.96 100.04) (end 170.95 100.03) (width 0.6) (layer F.Cu) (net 10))
 (segment (start 170.95 100.03) (end 170.95 98.45) (width 0.6) (layer F.Cu) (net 10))
 (segment (start 163.61 82.695058) (end 163.61 79.53) (width 0.6) (layer F.Cu) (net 1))
 (segment (start 160.935067 85.369991) (end 163.61 82.695058) (width 0.6) (layer F.Cu) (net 1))
 (segment (start 160.164419 85.369991) (end 160.935067 85.369991) (width 0.6) (layer F.Cu) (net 1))
 (segment (start 155.19 88.33) (end 157.20441 88.33) (width 0.6) (layer F.Cu) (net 1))
 (segment (start 157.20441 88.33) (end 160.164419 85.369991) (width 0.6) (layer F.Cu) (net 1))
 (segment (start 179.83 92.315) (end 178.38 92.315) (width 0.6) (layer F.Cu) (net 11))
 (segment (start 180.230001 92.715001) (end 179.83 92.315) (width 0.6) (layer F.Cu) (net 11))
 (segment (start 180.230001 100.832001) (end 180.230001 92.715001) (width 0.6) (layer F.Cu) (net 11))
 (segment (start 179.372001 101.690001) (end 180.230001 100.832001) (width 0.6) (layer F.Cu) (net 11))
 (segment (start 175.150001 101.690001) (end 179.372001 101.690001) (width 0.6) (layer F.Cu) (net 11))
 (segment (start 173.5 100.04) (end 175.150001 101.690001) (width 0.6) (layer F.Cu) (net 11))
 (segment (start 176.93 92.315) (end 178.38 92.315) (width 0.6) (layer F.Cu) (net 11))
 (segment (start 174.930022 90.315022) (end 176.93 92.315) (width 0.6) (layer F.Cu) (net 11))
 (segment (start 174.930022 89.168721) (end 174.930022 90.315022) (width 0.6) (layer F.Cu) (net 11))
 (segment (start 172.876301 87.115) (end 174.930022 89.168721) (width 0.6) (layer F.Cu) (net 11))
 (segment (start 169.3 87.115) (end 172.876301 87.115) (width 0.6) (layer F.Cu) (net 11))
 (segment (start 176.93 89.595) (end 176.93 90.12) (width 0.6) (layer F.Cu) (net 4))
 (segment (start 174.75 87.415) (end 176.93 89.595) (width 0.6) (layer F.Cu) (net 4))
 (segment (start 177.855 91.045) (end 178.38 91.045) (width 0.6) (layer F.Cu) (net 4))
 (segment (start 174.75 85.53) (end 174.75 87.415) (width 0.6) (layer F.Cu) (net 4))
 (segment (start 176.93 90.12) (end 177.855 91.045) (width 0.6) (layer F.Cu) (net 4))
 (segment (start 179.83 91.045) (end 178.38 91.045) (width 0.6) (layer F.Cu) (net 4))
 (segment (start 180.115649 91.045) (end 179.83 91.045) (width 0.6) (layer F.Cu) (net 4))
 (segment (start 181.330011 92.259362) (end 180.115649 91.045) (width 0.6) (layer F.Cu) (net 4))
 (segment (start 181.330011 101.28764) (end 181.330011 92.259362) (width 0.6) (layer F.Cu) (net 4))
 (segment (start 179.82764 102.790011) (end 181.330011 101.28764) (width 0.6) (layer F.Cu) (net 4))
 (segment (start 161.010011 102.790011) (end 179.82764 102.790011) (width 0.6) (layer F.Cu) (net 4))
 (segment (start 158.26 100.04) (end 161.010011 102.790011) (width 0.6) (layer F.Cu) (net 4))
 (segment (start 163.025 93.355) (end 164.08 92.3) (width 0.6) (layer F.Cu) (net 4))
 (segment (start 163.025 94.3) (end 163.025 93.355) (width 0.6) (layer F.Cu) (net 4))
 (segment (start 159.95 89.7) (end 159.65 89.7) (width 0.6) (layer F.Cu) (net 4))
 (segment (start 164.08 92.3) (end 162.55 92.3) (width 0.6) (layer F.Cu) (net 4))
 (segment (start 162.55 92.3) (end 159.95 89.7) (width 0.6) (layer F.Cu) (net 4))
 (segment (start 170.6 79.54) (end 170.61 79.53) (width 0.6) (layer F.Cu) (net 4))
 (segment (start 170.6 82.19) (end 170.6 79.54) (width 0.6) (layer F.Cu) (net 4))
 (segment (start 174.75 85.53) (end 173.94 85.53) (width 0.6) (layer F.Cu) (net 4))
 (segment (start 173.94 85.53) (end 170.6 82.19) (width 0.6) (layer F.Cu) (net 4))
 (segment (start 161.768372 96.156628) (end 161.145 96.78) (width 0.6) (layer F.Cu) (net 4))
 (segment (start 161.768372 95.946686) (end 161.768372 96.156628) (width 0.6) (layer F.Cu) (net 4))
 (segment (start 162.401628 95.31343) (end 161.768372 95.946686) (width 0.6) (layer F.Cu) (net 4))
 (segment (start 162.401628 94.923372) (end 162.401628 95.31343) (width 0.6) (layer F.Cu) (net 4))
 (segment (start 163.025 94.3) (end 162.401628 94.923372) (width 0.6) (layer F.Cu) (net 4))
 (segment (start 161.145 97.155) (end 158.26 100.04) (width 0.6) (layer F.Cu) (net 4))
 (segment (start 161.145 96.78) (end 161.145 97.155) (width 0.6) (layer F.Cu) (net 4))
 (segment (start 164.89 96.76) (end 164.91 96.78) (width 0.6) (layer F.Cu) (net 6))
 (segment (start 163.285 96.76) (end 164.89 96.76) (width 0.6) (layer F.Cu) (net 6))
 (segment (start 158.14 93.26) (end 159.65 91.75) (width 0.6) (layer F.Cu) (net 5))
 (segment (start 158.14 93.53) (end 158.14 93.26) (width 0.6) (layer F.Cu) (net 5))
 (segment (start 177.855 94.855) (end 178.38 94.855) (width 0.6) (layer F.Cu) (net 9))
 (segment (start 176.04 96.67) (end 177.855 94.855) (width 0.6) (layer F.Cu) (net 9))
 (segment (start 176.04 100.04) (end 176.04 96.67) (width 0.6) (layer F.Cu) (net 9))
 (segment (start 169.63 91.045) (end 171.08 91.045) (width 0.6) (layer F.Cu) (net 12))
 (segment (start 164.990001 98.389999) (end 165.974351 98.389999) (width 0.6) (layer F.Cu) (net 12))
 (segment (start 163.34 100.04) (end 164.990001 98.389999) (width 0.6) (layer F.Cu) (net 12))
 (segment (start 169.624979 91.050021) (end 169.63 91.045) (width 0.6) (layer F.Cu) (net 12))
 (segment (start 165.974351 98.389999) (end 166.25 98.11435) (width 0.6) (layer F.Cu) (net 12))
 (segment (start 166.25 98.11435) (end 166.25 94.025654) (width 0.6) (layer F.Cu) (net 12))
 (segment (start 166.25 94.025654) (end 169.225633 91.050021) (width 0.6) (layer F.Cu) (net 12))
 (segment (start 169.225633 91.050021) (end 169.624979 91.050021) (width 0.6) (layer F.Cu) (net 12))
 (segment (start 169.63 92.315) (end 171.08 92.315) (width 0.6) (layer F.Cu) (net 7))
 (segment (start 169.516302 92.315) (end 169.63 92.315) (width 0.6) (layer F.Cu) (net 7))
 (segment (start 167.71 94.121302) (end 169.516302 92.315) (width 0.6) (layer F.Cu) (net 7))
 (segment (start 167.71 96.78) (end 167.71 94.121302) (width 0.6) (layer F.Cu) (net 7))
 (segment (start 167.71 98.21) (end 167.71 96.78) (width 0.6) (layer F.Cu) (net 7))
 (segment (start 165.88 100.04) (end 167.71 98.21) (width 0.6) (layer F.Cu) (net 7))
 (segment (start 168.42 100.04) (end 169.429999 99.030001) (width 0.6) (layer F.Cu) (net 13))
 (segment (start 169.429999 99.030001) (end 169.429999 93.956955) (width 0.6) (layer F.Cu) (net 13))
 (segment (start 169.801954 93.585) (end 171.08 93.585) (width 0.6) (layer F.Cu) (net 13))
 (segment (start 169.429999 93.956955) (end 169.801954 93.585) (width 0.6) (layer F.Cu) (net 13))
 (segment (start 164.08 86.535) (end 164.145 86.47) (width 0.6) (layer F.Cu) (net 3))
 (segment (start 164.08 89) (end 164.08 86.535) (width 0.6) (layer F.Cu) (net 3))
 (segment (start 166.53 86.47) (end 166.575 86.425) (width 0.6) (layer F.Cu) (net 3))
 (segment (start 166.575 86.425) (end 166.34 86.19) (width 0.6) (layer F.Cu) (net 3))
 (segment (start 166.13 80.05) (end 166.11 80.03) (width 0.6) (layer F.Cu) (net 3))
 (segment (start 166.37 86.375) (end 166.13 86.135) (width 0.6) (layer F.Cu) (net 3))
 (segment (start 166.13 86.135) (end 166.13 80.05) (width 0.6) (layer F.Cu) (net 3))
 (segment (start 166.235 86.51) (end 166.37 86.375) (width 0.6) (layer F.Cu) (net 3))
 (segment (start 164.165 86.51) (end 166.235 86.51) (width 0.6) (layer F.Cu) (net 3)))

